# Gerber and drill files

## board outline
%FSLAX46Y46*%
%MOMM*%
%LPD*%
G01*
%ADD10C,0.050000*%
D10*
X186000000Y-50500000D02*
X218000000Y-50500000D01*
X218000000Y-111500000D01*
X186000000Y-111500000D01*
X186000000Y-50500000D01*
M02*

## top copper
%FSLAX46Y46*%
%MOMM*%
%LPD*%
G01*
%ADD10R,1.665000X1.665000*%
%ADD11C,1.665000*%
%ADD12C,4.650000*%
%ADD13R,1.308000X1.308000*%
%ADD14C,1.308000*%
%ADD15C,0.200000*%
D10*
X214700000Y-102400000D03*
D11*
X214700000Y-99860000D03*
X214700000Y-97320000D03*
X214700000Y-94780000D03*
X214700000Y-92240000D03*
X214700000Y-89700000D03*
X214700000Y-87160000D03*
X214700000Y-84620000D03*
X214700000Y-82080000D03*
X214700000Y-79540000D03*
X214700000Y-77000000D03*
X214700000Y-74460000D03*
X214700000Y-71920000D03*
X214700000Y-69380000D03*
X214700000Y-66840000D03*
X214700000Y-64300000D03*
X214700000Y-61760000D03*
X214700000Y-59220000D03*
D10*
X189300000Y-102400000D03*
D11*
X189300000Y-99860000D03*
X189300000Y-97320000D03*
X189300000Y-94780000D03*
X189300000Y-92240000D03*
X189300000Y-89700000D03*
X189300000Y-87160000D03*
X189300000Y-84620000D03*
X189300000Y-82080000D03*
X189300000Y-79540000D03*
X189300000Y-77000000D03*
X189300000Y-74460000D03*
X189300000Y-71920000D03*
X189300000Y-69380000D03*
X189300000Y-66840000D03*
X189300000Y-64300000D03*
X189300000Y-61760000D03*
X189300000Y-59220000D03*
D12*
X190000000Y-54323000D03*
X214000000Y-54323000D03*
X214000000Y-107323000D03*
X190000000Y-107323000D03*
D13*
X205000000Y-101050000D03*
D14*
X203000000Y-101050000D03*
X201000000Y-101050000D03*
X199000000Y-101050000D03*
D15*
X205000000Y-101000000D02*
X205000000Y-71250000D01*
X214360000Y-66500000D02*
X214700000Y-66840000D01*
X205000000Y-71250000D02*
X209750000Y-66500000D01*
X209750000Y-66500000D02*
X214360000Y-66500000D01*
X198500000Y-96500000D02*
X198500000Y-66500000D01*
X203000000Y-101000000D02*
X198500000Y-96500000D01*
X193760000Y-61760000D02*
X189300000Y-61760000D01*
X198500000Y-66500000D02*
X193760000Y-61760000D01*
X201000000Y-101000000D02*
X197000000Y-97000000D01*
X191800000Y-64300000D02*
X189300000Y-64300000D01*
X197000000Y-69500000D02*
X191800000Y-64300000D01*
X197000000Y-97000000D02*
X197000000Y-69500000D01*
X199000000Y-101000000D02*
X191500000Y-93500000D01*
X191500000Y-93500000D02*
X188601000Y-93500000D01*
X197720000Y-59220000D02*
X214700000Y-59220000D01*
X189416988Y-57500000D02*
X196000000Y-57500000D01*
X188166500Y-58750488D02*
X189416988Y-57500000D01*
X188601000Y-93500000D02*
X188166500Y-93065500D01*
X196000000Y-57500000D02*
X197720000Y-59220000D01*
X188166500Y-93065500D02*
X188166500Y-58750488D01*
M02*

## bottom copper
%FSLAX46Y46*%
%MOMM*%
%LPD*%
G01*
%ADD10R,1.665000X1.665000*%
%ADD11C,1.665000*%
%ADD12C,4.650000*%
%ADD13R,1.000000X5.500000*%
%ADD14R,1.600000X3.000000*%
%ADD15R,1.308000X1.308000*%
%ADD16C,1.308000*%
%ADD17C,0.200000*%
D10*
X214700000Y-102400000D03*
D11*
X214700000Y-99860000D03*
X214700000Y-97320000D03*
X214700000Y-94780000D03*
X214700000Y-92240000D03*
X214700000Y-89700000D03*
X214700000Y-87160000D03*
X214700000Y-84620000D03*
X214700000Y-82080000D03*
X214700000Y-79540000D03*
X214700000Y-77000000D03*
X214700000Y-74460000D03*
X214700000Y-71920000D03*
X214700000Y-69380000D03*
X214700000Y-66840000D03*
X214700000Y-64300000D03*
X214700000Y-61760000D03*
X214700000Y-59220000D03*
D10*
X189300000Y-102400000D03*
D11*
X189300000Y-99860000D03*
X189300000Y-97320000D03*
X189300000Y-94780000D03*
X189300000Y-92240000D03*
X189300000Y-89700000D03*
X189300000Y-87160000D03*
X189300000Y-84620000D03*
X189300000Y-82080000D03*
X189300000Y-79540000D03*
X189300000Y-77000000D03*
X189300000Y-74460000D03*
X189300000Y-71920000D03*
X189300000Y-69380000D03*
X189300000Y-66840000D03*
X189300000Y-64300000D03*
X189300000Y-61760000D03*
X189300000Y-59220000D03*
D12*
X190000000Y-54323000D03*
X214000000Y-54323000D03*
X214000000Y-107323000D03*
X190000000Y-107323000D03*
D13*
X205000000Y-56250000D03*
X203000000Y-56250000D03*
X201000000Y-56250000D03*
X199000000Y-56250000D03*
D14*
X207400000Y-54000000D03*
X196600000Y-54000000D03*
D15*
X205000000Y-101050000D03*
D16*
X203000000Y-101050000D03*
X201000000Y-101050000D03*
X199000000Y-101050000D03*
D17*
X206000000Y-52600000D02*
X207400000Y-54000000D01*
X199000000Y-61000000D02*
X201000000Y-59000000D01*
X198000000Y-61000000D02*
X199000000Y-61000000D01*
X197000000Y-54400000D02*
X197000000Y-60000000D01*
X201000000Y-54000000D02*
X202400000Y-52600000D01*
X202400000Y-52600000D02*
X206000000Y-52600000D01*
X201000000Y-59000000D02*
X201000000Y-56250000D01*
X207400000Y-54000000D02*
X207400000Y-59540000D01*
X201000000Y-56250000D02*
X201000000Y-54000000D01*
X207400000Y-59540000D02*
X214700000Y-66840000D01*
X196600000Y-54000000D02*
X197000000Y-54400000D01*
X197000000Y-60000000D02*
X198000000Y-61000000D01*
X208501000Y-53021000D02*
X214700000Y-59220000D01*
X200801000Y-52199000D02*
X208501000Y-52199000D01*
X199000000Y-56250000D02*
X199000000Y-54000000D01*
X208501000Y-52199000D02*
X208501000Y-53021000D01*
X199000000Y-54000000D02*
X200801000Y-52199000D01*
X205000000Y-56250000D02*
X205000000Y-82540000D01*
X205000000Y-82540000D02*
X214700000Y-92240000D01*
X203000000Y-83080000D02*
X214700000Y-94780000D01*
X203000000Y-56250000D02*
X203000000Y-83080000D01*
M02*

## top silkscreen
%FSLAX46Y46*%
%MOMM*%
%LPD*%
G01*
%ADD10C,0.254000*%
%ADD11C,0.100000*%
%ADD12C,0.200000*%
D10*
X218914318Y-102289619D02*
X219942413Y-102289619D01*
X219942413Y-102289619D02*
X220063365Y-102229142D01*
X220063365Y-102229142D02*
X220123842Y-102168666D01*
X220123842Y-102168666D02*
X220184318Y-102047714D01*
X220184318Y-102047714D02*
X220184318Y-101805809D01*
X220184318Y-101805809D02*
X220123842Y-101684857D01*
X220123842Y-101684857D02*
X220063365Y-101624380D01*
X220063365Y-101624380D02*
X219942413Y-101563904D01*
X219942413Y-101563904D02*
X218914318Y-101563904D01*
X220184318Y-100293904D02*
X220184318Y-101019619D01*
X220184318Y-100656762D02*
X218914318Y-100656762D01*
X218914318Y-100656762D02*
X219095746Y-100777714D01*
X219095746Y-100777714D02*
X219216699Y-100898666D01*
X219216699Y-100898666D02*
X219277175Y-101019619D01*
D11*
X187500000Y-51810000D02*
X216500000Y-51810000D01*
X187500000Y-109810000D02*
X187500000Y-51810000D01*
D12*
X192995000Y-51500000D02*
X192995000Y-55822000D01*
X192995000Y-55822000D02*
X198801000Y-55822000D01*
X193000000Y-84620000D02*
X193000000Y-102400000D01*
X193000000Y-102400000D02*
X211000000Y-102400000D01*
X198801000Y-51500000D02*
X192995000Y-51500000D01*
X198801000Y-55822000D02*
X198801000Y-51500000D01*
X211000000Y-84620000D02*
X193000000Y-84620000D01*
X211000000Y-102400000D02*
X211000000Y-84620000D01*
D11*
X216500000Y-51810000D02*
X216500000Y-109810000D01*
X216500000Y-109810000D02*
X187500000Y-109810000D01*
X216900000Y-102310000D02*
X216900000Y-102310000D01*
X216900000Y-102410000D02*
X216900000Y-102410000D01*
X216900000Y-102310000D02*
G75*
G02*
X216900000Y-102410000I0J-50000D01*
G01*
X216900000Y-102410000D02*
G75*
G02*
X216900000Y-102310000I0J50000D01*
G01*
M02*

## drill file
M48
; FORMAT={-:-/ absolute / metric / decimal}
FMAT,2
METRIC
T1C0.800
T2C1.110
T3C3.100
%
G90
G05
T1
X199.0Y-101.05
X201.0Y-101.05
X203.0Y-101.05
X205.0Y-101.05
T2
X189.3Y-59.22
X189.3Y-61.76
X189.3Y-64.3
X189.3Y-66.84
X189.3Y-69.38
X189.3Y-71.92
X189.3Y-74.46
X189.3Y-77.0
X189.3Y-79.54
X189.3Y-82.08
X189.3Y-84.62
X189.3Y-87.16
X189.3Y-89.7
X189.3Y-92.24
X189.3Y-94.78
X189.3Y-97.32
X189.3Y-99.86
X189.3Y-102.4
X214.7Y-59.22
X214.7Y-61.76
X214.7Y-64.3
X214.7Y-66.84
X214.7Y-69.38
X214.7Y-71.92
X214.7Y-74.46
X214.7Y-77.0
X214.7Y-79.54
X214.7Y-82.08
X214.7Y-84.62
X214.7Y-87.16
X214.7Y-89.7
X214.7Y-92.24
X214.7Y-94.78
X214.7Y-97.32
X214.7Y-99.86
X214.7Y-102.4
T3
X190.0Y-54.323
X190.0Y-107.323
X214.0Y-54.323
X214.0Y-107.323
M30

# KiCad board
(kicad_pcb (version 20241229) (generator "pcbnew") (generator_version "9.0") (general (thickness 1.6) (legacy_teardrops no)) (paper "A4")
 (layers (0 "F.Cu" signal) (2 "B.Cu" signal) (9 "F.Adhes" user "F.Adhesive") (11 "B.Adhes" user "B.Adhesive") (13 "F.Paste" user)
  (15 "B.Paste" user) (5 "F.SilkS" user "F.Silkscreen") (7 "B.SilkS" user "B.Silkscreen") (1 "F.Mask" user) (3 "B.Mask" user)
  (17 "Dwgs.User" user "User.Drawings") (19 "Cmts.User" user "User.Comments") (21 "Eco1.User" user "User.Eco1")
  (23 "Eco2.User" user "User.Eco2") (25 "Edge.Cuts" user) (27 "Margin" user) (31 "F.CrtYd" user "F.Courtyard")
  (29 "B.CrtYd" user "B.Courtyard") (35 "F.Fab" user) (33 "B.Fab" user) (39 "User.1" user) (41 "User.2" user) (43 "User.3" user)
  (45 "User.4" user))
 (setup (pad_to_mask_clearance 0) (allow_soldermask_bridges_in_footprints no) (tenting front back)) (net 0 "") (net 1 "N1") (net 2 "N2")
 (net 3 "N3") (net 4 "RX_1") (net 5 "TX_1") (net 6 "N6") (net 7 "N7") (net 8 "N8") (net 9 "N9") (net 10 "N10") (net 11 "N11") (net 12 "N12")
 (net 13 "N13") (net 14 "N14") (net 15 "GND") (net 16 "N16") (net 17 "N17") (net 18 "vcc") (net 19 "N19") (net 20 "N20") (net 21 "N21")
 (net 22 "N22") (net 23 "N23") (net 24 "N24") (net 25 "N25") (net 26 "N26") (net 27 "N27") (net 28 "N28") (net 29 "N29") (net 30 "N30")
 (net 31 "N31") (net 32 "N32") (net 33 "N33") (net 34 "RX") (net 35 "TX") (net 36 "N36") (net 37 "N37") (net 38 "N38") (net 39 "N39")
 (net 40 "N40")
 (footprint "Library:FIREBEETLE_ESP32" (layer "F.Cu") (at 202 77 -90)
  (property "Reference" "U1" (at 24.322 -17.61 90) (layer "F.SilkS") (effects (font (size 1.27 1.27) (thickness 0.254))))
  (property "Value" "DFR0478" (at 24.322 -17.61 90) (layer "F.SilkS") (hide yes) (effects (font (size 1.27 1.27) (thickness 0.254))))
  (fp_line (start -25.19 14.5) (end -25.19 -14.5) (stroke (width 0.1) (type solid)) (layer "F.SilkS"))
  (fp_line (start 32.81 14.5) (end -25.19 14.5) (stroke (width 0.1) (type solid)) (layer "F.SilkS"))
  (fp_line (start -25.5 9.005) (end -21.178 9.005) (stroke (width 0.2) (type solid)) (layer "F.SilkS"))
  (fp_line (start -21.178 9.005) (end -21.178 3.199) (stroke (width 0.2) (type solid)) (layer "F.SilkS"))
  (fp_line (start 7.62 9) (end 25.4 9) (stroke (width 0.2) (type solid)) (layer "F.SilkS"))
  (fp_line (start 25.4 9) (end 25.4 -9) (stroke (width 0.2) (type solid)) (layer "F.SilkS"))
  (fp_line (start -25.5 3.199) (end -25.5 9.005) (stroke (width 0.2) (type solid)) (layer "F.SilkS"))
  (fp_line (start -21.178 3.199) (end -25.5 3.199) (stroke (width 0.2) (type solid)) (layer "F.SilkS"))
  (fp_line (start 7.62 -9) (end 7.62 9) (stroke (width 0.2) (type solid)) (layer "F.SilkS"))
  (fp_line (start 25.4 -9) (end 7.62 -9) (stroke (width 0.2) (type solid)) (layer "F.SilkS"))
  (fp_line (start -25.19 -14.5) (end 32.81 -14.5) (stroke (width 0.1) (type solid)) (layer "F.SilkS"))
  (fp_line (start 32.81 -14.5) (end 32.81 14.5) (stroke (width 0.1) (type solid)) (layer "F.SilkS"))
  (fp_line (start 25.31 -14.9) (end 25.31 -14.9) (stroke (width 0.1) (type solid)) (layer "F.SilkS"))
  (fp_line (start 25.41 -14.9) (end 25.41 -14.9) (stroke (width 0.1) (type solid)) (layer "F.SilkS"))
  (fp_arc (start 25.31 -14.9) (mid 25.36 -14.95) (end 25.41 -14.9) (stroke (width 0.1) (type solid)) (layer "F.SilkS"))
  (fp_arc (start 25.41 -14.9) (mid 25.36 -14.85) (end 25.31 -14.9) (stroke (width 0.1) (type solid)) (layer "F.SilkS"))
  (pad "1" thru_hole rect (at 25.4 -12.7 270) (size 1.665 1.665) (drill 1.11) (layers "*.Cu" "*.Mask") (remove_unused_layers no)
   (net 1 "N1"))
  (pad "2" thru_hole circle (at 22.86 -12.7 270) (size 1.665 1.665) (drill 1.11) (layers "*.Cu" "*.Mask") (remove_unused_layers no)
   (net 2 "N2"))
  (pad "3" thru_hole circle (at 20.32 -12.7 270) (size 1.665 1.665) (drill 1.11) (layers "*.Cu" "*.Mask") (remove_unused_layers no)
   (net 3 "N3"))
  (pad "4" thru_hole circle (at 17.78 -12.7 270) (size 1.665 1.665) (drill 1.11) (layers "*.Cu" "*.Mask") (remove_unused_layers no)
   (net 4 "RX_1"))
  (pad "5" thru_hole circle (at 15.24 -12.7 270) (size 1.665 1.665) (drill 1.11) (layers "*.Cu" "*.Mask") (remove_unused_layers no)
   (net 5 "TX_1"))
  (pad "6" thru_hole circle (at 12.7 -12.7 270) (size 1.665 1.665) (drill 1.11) (layers "*.Cu" "*.Mask") (remove_unused_layers no)
   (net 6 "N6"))
  (pad "7" thru_hole circle (at 10.16 -12.7 270) (size 1.665 1.665) (drill 1.11) (layers "*.Cu" "*.Mask") (remove_unused_layers no)
   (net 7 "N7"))
  (pad "8" thru_hole circle (at 7.62 -12.7 270) (size 1.665 1.665) (drill 1.11) (layers "*.Cu" "*.Mask") (remove_unused_layers no)
   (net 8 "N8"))
  (pad "9" thru_hole circle (at 5.08 -12.7 270) (size 1.665 1.665) (drill 1.11) (layers "*.Cu" "*.Mask") (remove_unused_layers no)
   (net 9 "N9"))
  (pad "10" thru_hole circle (at 2.54 -12.7 270) (size 1.665 1.665) (drill 1.11) (layers "*.Cu" "*.Mask") (remove_unused_layers no)
   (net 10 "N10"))
  (pad "11" thru_hole circle (at 0 -12.7 270) (size 1.665 1.665) (drill 1.11) (layers "*.Cu" "*.Mask") (remove_unused_layers no)
   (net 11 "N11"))
  (pad "12" thru_hole circle (at -2.54 -12.7 270) (size 1.665 1.665) (drill 1.11) (layers "*.Cu" "*.Mask") (remove_unused_layers no)
   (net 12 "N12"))
  (pad "13" thru_hole circle (at -5.08 -12.7 270) (size 1.665 1.665) (drill 1.11) (layers "*.Cu" "*.Mask") (remove_unused_layers no)
   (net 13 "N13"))
  (pad "14" thru_hole circle (at -7.62 -12.7 270) (size 1.665 1.665) (drill 1.11) (layers "*.Cu" "*.Mask") (remove_unused_layers no)
   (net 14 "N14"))
  (pad "15" thru_hole circle (at -10.16 -12.7 270) (size 1.665 1.665) (drill 1.11) (layers "*.Cu" "*.Mask") (remove_unused_layers no)
   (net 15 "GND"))
  (pad "16" thru_hole circle (at -12.7 -12.7 270) (size 1.665 1.665) (drill 1.11) (layers "*.Cu" "*.Mask") (remove_unused_layers no)
   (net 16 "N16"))
  (pad "17" thru_hole circle (at -15.24 -12.7 270) (size 1.665 1.665) (drill 1.11) (layers "*.Cu" "*.Mask") (remove_unused_layers no)
   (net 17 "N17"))
  (pad "18" thru_hole circle (at -17.78 -12.7 270) (size 1.665 1.665) (drill 1.11) (layers "*.Cu" "*.Mask") (remove_unused_layers no)
   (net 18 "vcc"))
  (pad "19" thru_hole rect (at 25.4 12.7 270) (size 1.665 1.665) (drill 1.11) (layers "*.Cu" "*.Mask") (remove_unused_layers no)
   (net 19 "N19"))
  (pad "20" thru_hole circle (at 22.86 12.7 270) (size 1.665 1.665) (drill 1.11) (layers "*.Cu" "*.Mask") (remove_unused_layers no)
   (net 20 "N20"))
  (pad "21" thru_hole circle (at 20.32 12.7 270) (size 1.665 1.665) (drill 1.11) (layers "*.Cu" "*.Mask") (remove_unused_layers no)
   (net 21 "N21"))
  (pad "22" thru_hole circle (at 17.78 12.7 270) (size 1.665 1.665) (drill 1.11) (layers "*.Cu" "*.Mask") (remove_unused_layers no)
   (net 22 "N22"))
  (pad "23" thru_hole circle (at 15.24 12.7 270) (size 1.665 1.665) (drill 1.11) (layers "*.Cu" "*.Mask") (remove_unused_layers no)
   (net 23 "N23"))
  (pad "24" thru_hole circle (at 12.7 12.7 270) (size 1.665 1.665) (drill 1.11) (layers "*.Cu" "*.Mask") (remove_unused_layers no)
   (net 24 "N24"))
  (pad "25" thru_hole circle (at 10.16 12.7 270) (size 1.665 1.665) (drill 1.11) (layers "*.Cu" "*.Mask") (remove_unused_layers no)
   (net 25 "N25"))
  (pad "26" thru_hole circle (at 7.62 12.7 270) (size 1.665 1.665) (drill 1.11) (layers "*.Cu" "*.Mask") (remove_unused_layers no)
   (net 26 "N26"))
  (pad "27" thru_hole circle (at 5.08 12.7 270) (size 1.665 1.665) (drill 1.11) (layers "*.Cu" "*.Mask") (remove_unused_layers no)
   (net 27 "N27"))
  (pad "28" thru_hole circle (at 2.54 12.7 270) (size 1.665 1.665) (drill 1.11) (layers "*.Cu" "*.Mask") (remove_unused_layers no)
   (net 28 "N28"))
  (pad "29" thru_hole circle (at 0 12.7 270) (size 1.665 1.665) (drill 1.11) (layers "*.Cu" "*.Mask") (remove_unused_layers no)
   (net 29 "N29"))
  (pad "30" thru_hole circle (at -2.54 12.7 270) (size 1.665 1.665) (drill 1.11) (layers "*.Cu" "*.Mask") (remove_unused_layers no)
   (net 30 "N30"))
  (pad "31" thru_hole circle (at -5.08 12.7 270) (size 1.665 1.665) (drill 1.11) (layers "*.Cu" "*.Mask") (remove_unused_layers no)
   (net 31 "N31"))
  (pad "32" thru_hole circle (at -7.62 12.7 270) (size 1.665 1.665) (drill 1.11) (layers "*.Cu" "*.Mask") (remove_unused_layers no)
   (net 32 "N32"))
  (pad "33" thru_hole circle (at -10.16 12.7 270) (size 1.665 1.665) (drill 1.11) (layers "*.Cu" "*.Mask") (remove_unused_layers no)
   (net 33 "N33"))
  (pad "34" thru_hole circle (at -12.7 12.7 270) (size 1.665 1.665) (drill 1.11) (layers "*.Cu" "*.Mask") (remove_unused_layers no)
   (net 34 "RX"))
  (pad "35" thru_hole circle (at -15.24 12.7 270) (size 1.665 1.665) (drill 1.11) (layers "*.Cu" "*.Mask") (remove_unused_layers no)
   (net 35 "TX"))
  (pad "36" thru_hole circle (at -17.78 12.7 270) (size 1.665 1.665) (drill 1.11) (layers "*.Cu" "*.Mask") (remove_unused_layers no)
   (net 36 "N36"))
  (pad "MH1" thru_hole circle (at -22.677 12 270) (size 4.65 4.65) (drill 3.1) (layers "*.Cu" "*.Mask") (remove_unused_layers no)
   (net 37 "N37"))
  (pad "MH2" thru_hole circle (at -22.677 -12 270) (size 4.65 4.65) (drill 3.1) (layers "*.Cu" "*.Mask") (remove_unused_layers no)
   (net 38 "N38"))
  (pad "MH3" thru_hole circle (at 30.323 -12 270) (size 4.65 4.65) (drill 3.1) (layers "*.Cu" "*.Mask") (remove_unused_layers no)
   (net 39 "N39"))
  (pad "MH4" thru_hole circle (at 30.323 12 270) (size 4.65 4.65) (drill 3.1) (layers "*.Cu" "*.Mask") (remove_unused_layers no)
   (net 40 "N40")))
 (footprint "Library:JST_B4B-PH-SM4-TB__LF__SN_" (layer "B.Cu") (at 202 54 180)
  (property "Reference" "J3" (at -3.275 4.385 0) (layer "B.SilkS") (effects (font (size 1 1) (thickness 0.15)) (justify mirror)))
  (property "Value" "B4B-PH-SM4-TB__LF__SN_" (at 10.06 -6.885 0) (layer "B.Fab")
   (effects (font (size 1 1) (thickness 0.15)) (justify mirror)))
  (pad "1" smd rect (at -3 -2.25 180) (size 1 5.5) (layers "B.Cu" "B.Mask" "B.Paste") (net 5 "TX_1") (solder_mask_margin 0.102))
  (pad "2" smd rect (at -1 -2.25 180) (size 1 5.5) (layers "B.Cu" "B.Mask" "B.Paste") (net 4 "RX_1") (solder_mask_margin 0.102))
  (pad "3" smd rect (at 1 -2.25 180) (size 1 5.5) (layers "B.Cu" "B.Mask" "B.Paste") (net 15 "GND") (solder_mask_margin 0.102))
  (pad "4" smd rect (at 3 -2.25 180) (size 1 5.5) (layers "B.Cu" "B.Mask" "B.Paste") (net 18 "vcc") (solder_mask_margin 0.102))
  (pad "SH1" smd rect (at -5.4 0 180) (size 1.6 3) (layers "B.Cu" "B.Mask" "B.Paste") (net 15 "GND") (solder_mask_margin 0.102))
  (pad "SH2" smd rect (at 5.4 0 180) (size 1.6 3) (layers "B.Cu" "B.Mask" "B.Paste") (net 15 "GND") (solder_mask_margin 0.102)))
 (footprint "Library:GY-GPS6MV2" (layer "B.Cu") (at 202 84)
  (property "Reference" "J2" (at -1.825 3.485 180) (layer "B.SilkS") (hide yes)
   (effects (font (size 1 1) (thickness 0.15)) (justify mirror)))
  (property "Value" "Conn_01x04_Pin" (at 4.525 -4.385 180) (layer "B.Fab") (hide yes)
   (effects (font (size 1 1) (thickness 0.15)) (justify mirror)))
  (pad "1" thru_hole rect (at 3 17.05 180) (size 1.308 1.308) (drill 0.8) (layers "*.Cu" "*.Mask") (remove_unused_layers no) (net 15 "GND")
   (solder_mask_margin 0.102))
  (pad "2" thru_hole circle (at 1 17.05 180) (size 1.308 1.308) (drill 0.8) (layers "*.Cu" "*.Mask") (remove_unused_layers no) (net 35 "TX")
   (solder_mask_margin 0.102))
  (pad "3" thru_hole circle (at -1 17.05 180) (size 1.308 1.308) (drill 0.8) (layers "*.Cu" "*.Mask") (remove_unused_layers no)
   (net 34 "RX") (solder_mask_margin 0.102))
  (pad "4" thru_hole circle (at -3 17.05 180) (size 1.308 1.308) (drill 0.8) (layers "*.Cu" "*.Mask") (remove_unused_layers no)
   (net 18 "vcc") (solder_mask_margin 0.102)))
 (gr_rect (start 186 50.5) (end 218 111.5) (stroke (width 0.05) (type default)) (fill no) (layer "Edge.Cuts"))
 (segment (start 205 101) (end 205 71.25) (width 0.2) (layer "F.Cu") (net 15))
 (segment (start 214.36 66.5) (end 214.7 66.84) (width 0.2) (layer "F.Cu") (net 15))
 (segment (start 205 71.25) (end 209.75 66.5) (width 0.2) (layer "F.Cu") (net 15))
 (segment (start 209.75 66.5) (end 214.36 66.5) (width 0.2) (layer "F.Cu") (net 15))
 (segment (start 206 52.6) (end 207.4 54) (width 0.2) (layer "B.Cu") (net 15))
 (segment (start 199 61) (end 201 59) (width 0.2) (layer "B.Cu") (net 15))
 (segment (start 198 61) (end 199 61) (width 0.2) (layer "B.Cu") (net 15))
 (segment (start 197 54.4) (end 197 60) (width 0.2) (layer "B.Cu") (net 15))
 (segment (start 201 54) (end 202.4 52.6) (width 0.2) (layer "B.Cu") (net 15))
 (segment (start 202.4 52.6) (end 206 52.6) (width 0.2) (layer "B.Cu") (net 15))
 (segment (start 201 59) (end 201 56.25) (width 0.2) (layer "B.Cu") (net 15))
 (segment (start 207.4 54) (end 207.4 59.54) (width 0.2) (layer "B.Cu") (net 15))
 (segment (start 201 56.25) (end 201 54) (width 0.2) (layer "B.Cu") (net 15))
 (segment (start 207.4 59.54) (end 214.7 66.84) (width 0.2) (layer "B.Cu") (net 15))
 (segment (start 196.6 54) (end 197 54.4) (width 0.2) (layer "B.Cu") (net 15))
 (segment (start 197 60) (end 198 61) (width 0.2) (layer "B.Cu") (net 15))
 (segment (start 198.5 96.5) (end 198.5 66.5) (width 0.2) (layer "F.Cu") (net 35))
 (segment (start 203 101) (end 198.5 96.5) (width 0.2) (layer "F.Cu") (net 35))
 (segment (start 193.76 61.76) (end 189.3 61.76) (width 0.2) (layer "F.Cu") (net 35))
 (segment (start 198.5 66.5) (end 193.76 61.76) (width 0.2) (layer "F.Cu") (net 35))
 (segment (start 201 101) (end 197 97) (width 0.2) (layer "F.Cu") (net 34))
 (segment (start 191.8 64.3) (end 189.3 64.3) (width 0.2) (layer "F.Cu") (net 34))
 (segment (start 197 69.5) (end 191.8 64.3) (width 0.2) (layer "F.Cu") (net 34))
 (segment (start 197 97) (end 197 69.5) (width 0.2) (layer "F.Cu") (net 34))
 (segment (start 199 101) (end 191.5 93.5) (width 0.2) (layer "F.Cu") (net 18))
 (segment (start 191.5 93.5) (end 188.601 93.5) (width 0.2) (layer "F.Cu") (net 18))
 (segment (start 197.72 59.22) (end 214.7 59.22) (width 0.2) (layer "F.Cu") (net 18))
 (segment (start 189.416988 57.5) (end 196 57.5) (width 0.2) (layer "F.Cu") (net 18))
 (segment (start 188.1665 58.750488) (end 189.416988 57.5) (width 0.2) (layer "F.Cu") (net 18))
 (segment (start 188.601 93.5) (end 188.1665 93.0655) (width 0.2) (layer "F.Cu") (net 18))
 (segment (start 196 57.5) (end 197.72 59.22) (width 0.2) (layer "F.Cu") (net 18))
 (segment (start 188.1665 93.0655) (end 188.1665 58.750488) (width 0.2) (layer "F.Cu") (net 18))
 (segment (start 208.501 53.021) (end 214.7 59.22) (width 0.2) (layer "B.Cu") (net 18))
 (segment (start 200.801 52.199) (end 208.501 52.199) (width 0.2) (layer "B.Cu") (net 18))
 (segment (start 199 56.25) (end 199 54) (width 0.2) (layer "B.Cu") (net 18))
 (segment (start 208.501 52.199) (end 208.501 53.021) (width 0.2) (layer "B.Cu") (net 18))
 (segment (start 199 54) (end 200.801 52.199) (width 0.2) (layer "B.Cu") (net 18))
 (segment (start 205 56.25) (end 205 82.54) (width 0.2) (layer "B.Cu") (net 5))
 (segment (start 205 82.54) (end 214.7 92.24) (width 0.2) (layer "B.Cu") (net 5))
 (segment (start 203 83.08) (end 214.7 94.78) (width 0.2) (layer "B.Cu") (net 4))
 (segment (start 203 56.25) (end 203 83.08) (width 0.2) (layer "B.Cu") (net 4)))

